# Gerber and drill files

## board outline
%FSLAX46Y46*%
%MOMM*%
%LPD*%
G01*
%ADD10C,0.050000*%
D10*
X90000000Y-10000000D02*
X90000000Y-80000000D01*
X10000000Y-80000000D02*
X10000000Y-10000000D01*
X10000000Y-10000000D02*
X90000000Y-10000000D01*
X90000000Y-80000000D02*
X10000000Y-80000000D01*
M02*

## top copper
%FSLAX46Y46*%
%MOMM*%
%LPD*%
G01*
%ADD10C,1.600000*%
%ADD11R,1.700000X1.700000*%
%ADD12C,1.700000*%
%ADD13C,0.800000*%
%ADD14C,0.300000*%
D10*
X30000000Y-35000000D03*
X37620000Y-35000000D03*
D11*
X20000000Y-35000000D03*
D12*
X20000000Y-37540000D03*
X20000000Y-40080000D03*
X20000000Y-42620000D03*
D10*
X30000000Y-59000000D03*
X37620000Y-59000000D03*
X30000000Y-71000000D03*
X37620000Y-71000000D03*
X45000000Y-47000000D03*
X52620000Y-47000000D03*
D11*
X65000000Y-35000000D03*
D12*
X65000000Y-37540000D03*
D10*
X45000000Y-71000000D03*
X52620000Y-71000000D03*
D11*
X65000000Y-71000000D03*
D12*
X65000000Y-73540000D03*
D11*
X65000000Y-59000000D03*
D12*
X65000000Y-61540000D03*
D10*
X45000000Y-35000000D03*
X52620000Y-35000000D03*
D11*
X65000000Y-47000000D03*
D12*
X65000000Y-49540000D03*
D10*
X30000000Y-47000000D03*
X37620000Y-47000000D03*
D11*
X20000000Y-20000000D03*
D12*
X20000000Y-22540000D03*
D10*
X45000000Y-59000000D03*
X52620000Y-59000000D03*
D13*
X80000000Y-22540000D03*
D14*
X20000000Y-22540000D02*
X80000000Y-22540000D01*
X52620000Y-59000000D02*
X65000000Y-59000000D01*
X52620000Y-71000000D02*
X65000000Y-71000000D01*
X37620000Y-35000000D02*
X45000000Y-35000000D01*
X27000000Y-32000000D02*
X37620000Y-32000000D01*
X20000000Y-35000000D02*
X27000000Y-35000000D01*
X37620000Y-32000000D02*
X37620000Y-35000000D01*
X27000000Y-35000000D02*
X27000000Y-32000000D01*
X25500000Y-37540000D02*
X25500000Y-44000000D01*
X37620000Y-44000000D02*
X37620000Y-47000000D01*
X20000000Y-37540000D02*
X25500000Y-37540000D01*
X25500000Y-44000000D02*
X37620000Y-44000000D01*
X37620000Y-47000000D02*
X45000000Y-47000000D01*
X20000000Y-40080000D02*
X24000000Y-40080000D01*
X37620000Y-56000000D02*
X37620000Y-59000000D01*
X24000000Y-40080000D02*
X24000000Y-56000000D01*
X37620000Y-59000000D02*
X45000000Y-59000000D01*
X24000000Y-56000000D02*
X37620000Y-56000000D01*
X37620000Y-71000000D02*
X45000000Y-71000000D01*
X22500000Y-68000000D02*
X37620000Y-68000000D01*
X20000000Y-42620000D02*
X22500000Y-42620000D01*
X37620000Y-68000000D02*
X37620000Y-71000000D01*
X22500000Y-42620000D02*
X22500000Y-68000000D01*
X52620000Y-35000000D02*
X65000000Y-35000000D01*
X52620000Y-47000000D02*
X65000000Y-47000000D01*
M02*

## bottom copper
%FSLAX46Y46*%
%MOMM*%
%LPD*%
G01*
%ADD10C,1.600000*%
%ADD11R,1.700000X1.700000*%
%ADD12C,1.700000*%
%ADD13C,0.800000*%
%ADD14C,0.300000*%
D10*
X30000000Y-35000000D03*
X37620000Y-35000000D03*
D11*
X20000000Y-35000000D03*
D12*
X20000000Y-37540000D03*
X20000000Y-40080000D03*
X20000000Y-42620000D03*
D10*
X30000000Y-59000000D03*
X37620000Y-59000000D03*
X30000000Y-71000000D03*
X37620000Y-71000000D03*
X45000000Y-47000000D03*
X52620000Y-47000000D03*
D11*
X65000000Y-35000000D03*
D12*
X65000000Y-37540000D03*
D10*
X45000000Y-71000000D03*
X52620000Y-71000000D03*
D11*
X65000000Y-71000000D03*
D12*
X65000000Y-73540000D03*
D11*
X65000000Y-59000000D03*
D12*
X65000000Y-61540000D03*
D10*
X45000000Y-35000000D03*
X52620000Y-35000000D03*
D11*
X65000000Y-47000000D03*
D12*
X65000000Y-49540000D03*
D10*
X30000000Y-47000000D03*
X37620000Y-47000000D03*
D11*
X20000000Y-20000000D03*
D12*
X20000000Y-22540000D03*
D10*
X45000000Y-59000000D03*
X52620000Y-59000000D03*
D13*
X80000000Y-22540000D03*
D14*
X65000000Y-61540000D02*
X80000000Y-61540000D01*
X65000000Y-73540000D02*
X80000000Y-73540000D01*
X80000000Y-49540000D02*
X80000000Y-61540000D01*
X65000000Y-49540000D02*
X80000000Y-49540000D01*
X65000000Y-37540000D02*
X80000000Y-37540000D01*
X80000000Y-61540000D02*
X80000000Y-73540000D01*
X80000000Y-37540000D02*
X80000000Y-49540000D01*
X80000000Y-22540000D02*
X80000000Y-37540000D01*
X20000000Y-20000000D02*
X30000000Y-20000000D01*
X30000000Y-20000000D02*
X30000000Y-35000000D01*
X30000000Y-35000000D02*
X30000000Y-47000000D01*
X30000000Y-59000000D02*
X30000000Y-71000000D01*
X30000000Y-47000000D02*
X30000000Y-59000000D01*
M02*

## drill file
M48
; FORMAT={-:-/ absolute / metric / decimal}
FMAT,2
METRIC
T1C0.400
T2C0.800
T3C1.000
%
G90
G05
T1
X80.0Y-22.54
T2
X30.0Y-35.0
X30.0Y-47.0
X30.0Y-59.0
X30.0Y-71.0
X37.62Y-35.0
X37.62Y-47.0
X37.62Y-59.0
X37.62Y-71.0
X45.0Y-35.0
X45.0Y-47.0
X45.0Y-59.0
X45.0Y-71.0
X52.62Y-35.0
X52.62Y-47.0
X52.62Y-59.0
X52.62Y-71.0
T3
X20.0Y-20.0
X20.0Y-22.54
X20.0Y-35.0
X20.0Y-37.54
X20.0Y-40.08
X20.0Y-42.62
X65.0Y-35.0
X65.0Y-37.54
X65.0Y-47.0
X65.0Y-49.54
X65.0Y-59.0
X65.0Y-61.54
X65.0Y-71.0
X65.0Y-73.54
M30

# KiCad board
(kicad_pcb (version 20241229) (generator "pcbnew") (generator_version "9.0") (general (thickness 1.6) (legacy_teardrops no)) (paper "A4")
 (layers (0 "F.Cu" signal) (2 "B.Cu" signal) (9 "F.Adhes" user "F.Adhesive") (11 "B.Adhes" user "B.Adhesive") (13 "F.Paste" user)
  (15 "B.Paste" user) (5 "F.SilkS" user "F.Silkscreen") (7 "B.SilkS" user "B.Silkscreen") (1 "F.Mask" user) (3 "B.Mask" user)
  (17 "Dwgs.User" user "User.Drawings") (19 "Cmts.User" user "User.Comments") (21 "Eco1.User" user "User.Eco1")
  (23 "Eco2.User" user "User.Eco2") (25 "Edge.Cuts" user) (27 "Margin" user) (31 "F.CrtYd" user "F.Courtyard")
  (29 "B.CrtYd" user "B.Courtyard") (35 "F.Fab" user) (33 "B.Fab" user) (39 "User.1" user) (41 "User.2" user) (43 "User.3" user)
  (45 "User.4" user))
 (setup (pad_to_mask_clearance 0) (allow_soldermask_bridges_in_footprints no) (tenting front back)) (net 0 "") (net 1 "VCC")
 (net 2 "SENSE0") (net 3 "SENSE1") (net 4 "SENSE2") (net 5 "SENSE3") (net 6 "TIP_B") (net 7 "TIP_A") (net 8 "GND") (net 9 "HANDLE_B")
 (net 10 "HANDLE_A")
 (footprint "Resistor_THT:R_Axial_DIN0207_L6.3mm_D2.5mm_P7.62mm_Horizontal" (layer "F.Cu") (at 30 35)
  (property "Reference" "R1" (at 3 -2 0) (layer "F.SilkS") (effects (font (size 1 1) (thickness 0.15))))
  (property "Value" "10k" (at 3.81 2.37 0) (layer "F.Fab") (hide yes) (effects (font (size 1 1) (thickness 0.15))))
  (pad "1" thru_hole circle (at 0 0) (size 1.6 1.6) (drill 0.8) (layers "*.Cu" "*.Mask") (remove_unused_layers no) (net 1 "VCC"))
  (pad "2" thru_hole circle (at 7.62 0) (size 1.6 1.6) (drill 0.8) (layers "*.Cu" "*.Mask") (remove_unused_layers no) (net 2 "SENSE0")))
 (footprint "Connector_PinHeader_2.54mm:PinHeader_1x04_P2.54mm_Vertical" (layer "F.Cu") (at 20 35)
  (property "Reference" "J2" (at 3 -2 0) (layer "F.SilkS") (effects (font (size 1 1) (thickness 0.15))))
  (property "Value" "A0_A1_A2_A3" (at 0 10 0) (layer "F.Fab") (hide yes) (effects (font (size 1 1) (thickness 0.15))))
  (pad "1" thru_hole rect (at 0 0) (size 1.7 1.7) (drill 1) (layers "*.Cu" "*.Mask") (remove_unused_layers no) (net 2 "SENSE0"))
  (pad "2" thru_hole circle (at 0 2.54) (size 1.7 1.7) (drill 1) (layers "*.Cu" "*.Mask") (remove_unused_layers no) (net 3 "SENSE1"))
  (pad "3" thru_hole circle (at 0 5.08) (size 1.7 1.7) (drill 1) (layers "*.Cu" "*.Mask") (remove_unused_layers no) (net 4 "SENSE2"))
  (pad "4" thru_hole circle (at 0 7.62) (size 1.7 1.7) (drill 1) (layers "*.Cu" "*.Mask") (remove_unused_layers no) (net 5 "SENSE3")))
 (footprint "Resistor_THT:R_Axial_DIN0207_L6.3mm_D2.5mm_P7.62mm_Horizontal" (layer "F.Cu") (at 30 59)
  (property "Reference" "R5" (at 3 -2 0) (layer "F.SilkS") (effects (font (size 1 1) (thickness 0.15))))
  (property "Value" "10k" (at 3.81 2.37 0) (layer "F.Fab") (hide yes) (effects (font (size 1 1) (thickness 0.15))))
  (pad "1" thru_hole circle (at 0 0) (size 1.6 1.6) (drill 0.8) (layers "*.Cu" "*.Mask") (remove_unused_layers no) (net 1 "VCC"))
  (pad "2" thru_hole circle (at 7.62 0) (size 1.6 1.6) (drill 0.8) (layers "*.Cu" "*.Mask") (remove_unused_layers no) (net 4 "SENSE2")))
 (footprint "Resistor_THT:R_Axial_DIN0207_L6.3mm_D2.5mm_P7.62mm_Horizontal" (layer "F.Cu") (at 30 71)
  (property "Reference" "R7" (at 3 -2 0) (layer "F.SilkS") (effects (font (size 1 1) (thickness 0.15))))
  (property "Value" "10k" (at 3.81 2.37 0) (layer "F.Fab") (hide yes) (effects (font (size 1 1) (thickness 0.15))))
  (pad "1" thru_hole circle (at 0 0) (size 1.6 1.6) (drill 0.8) (layers "*.Cu" "*.Mask") (remove_unused_layers no) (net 1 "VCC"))
  (pad "2" thru_hole circle (at 7.62 0) (size 1.6 1.6) (drill 0.8) (layers "*.Cu" "*.Mask") (remove_unused_layers no) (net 5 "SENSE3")))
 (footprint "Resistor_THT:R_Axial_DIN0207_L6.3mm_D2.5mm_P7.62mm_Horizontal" (layer "F.Cu") (at 45 47)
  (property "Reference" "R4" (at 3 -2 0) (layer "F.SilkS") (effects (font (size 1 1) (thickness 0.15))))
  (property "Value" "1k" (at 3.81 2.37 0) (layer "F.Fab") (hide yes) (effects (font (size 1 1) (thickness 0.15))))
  (pad "1" thru_hole circle (at 0 0) (size 1.6 1.6) (drill 0.8) (layers "*.Cu" "*.Mask") (remove_unused_layers no) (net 3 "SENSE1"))
  (pad "2" thru_hole circle (at 7.62 0) (size 1.6 1.6) (drill 0.8) (layers "*.Cu" "*.Mask") (remove_unused_layers no) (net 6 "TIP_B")))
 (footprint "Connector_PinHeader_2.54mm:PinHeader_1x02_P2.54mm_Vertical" (layer "F.Cu") (at 65 35)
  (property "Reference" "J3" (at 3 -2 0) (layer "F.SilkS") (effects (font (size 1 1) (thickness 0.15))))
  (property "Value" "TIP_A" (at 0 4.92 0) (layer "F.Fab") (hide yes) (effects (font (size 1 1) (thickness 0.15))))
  (pad "1" thru_hole rect (at 0 0) (size 1.7 1.7) (drill 1) (layers "*.Cu" "*.Mask") (remove_unused_layers no) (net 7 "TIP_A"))
  (pad "2" thru_hole circle (at 0 2.54) (size 1.7 1.7) (drill 1) (layers "*.Cu" "*.Mask") (remove_unused_layers no) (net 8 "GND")))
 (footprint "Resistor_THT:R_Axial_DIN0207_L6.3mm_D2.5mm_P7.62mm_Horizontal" (layer "F.Cu") (at 45 71)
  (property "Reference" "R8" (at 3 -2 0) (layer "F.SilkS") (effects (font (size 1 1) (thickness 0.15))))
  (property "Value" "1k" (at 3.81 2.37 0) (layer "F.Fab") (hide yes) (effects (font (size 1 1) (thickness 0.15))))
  (pad "1" thru_hole circle (at 0 0) (size 1.6 1.6) (drill 0.8) (layers "*.Cu" "*.Mask") (remove_unused_layers no) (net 5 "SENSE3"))
  (pad "2" thru_hole circle (at 7.62 0) (size 1.6 1.6) (drill 0.8) (layers "*.Cu" "*.Mask") (remove_unused_layers no) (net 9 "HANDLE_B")))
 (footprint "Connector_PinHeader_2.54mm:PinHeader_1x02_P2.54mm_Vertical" (layer "F.Cu") (at 65 71)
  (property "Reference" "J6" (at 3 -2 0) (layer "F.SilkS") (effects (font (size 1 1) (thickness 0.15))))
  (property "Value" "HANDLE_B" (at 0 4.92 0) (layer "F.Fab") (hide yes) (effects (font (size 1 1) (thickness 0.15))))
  (pad "1" thru_hole rect (at 0 0) (size 1.7 1.7) (drill 1) (layers "*.Cu" "*.Mask") (remove_unused_layers no) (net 9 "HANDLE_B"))
  (pad "2" thru_hole circle (at 0 2.54) (size 1.7 1.7) (drill 1) (layers "*.Cu" "*.Mask") (remove_unused_layers no) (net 8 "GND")))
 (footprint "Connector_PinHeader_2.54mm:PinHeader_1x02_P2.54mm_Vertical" (layer "F.Cu") (at 65 59)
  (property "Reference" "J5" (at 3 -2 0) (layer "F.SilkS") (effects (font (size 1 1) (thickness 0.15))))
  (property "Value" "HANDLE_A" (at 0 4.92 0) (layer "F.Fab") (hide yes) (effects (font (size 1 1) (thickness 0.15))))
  (pad "1" thru_hole rect (at 0 0) (size 1.7 1.7) (drill 1) (layers "*.Cu" "*.Mask") (remove_unused_layers no) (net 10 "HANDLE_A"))
  (pad "2" thru_hole circle (at 0 2.54) (size 1.7 1.7) (drill 1) (layers "*.Cu" "*.Mask") (remove_unused_layers no) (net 8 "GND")))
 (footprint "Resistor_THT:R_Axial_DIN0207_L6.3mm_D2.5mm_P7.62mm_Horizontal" (layer "F.Cu") (at 45 35)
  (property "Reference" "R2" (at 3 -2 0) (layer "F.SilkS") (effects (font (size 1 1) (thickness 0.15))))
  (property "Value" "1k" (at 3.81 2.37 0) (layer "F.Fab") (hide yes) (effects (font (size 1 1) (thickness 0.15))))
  (pad "1" thru_hole circle (at 0 0) (size 1.6 1.6) (drill 0.8) (layers "*.Cu" "*.Mask") (remove_unused_layers no) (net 2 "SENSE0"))
  (pad "2" thru_hole circle (at 7.62 0) (size 1.6 1.6) (drill 0.8) (layers "*.Cu" "*.Mask") (remove_unused_layers no) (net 7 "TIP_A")))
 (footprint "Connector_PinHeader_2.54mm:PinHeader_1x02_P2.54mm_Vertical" (layer "F.Cu") (at 65 47)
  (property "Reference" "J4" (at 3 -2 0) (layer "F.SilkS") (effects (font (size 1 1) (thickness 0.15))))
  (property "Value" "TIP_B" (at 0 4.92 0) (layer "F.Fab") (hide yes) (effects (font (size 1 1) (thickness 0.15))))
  (pad "1" thru_hole rect (at 0 0) (size 1.7 1.7) (drill 1) (layers "*.Cu" "*.Mask") (remove_unused_layers no) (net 6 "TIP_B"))
  (pad "2" thru_hole circle (at 0 2.54) (size 1.7 1.7) (drill 1) (layers "*.Cu" "*.Mask") (remove_unused_layers no) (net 8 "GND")))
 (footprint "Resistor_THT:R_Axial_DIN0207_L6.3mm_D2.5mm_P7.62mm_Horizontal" (layer "F.Cu") (at 30 47)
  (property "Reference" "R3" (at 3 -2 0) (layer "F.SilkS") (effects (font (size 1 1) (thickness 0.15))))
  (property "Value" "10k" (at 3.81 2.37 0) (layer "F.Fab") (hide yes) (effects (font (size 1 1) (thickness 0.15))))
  (pad "1" thru_hole circle (at 0 0) (size 1.6 1.6) (drill 0.8) (layers "*.Cu" "*.Mask") (remove_unused_layers no) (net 1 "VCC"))
  (pad "2" thru_hole circle (at 7.62 0) (size 1.6 1.6) (drill 0.8) (layers "*.Cu" "*.Mask") (remove_unused_layers no) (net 3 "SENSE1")))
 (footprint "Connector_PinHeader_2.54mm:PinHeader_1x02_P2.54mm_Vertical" (layer "F.Cu") (at 20 20)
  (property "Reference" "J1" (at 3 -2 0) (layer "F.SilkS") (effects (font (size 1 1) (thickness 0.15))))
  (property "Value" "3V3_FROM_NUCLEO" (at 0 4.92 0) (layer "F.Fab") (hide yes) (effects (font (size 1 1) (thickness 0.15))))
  (pad "1" thru_hole rect (at 0 0) (size 1.7 1.7) (drill 1) (layers "*.Cu" "*.Mask") (remove_unused_layers no) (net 1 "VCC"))
  (pad "2" thru_hole circle (at 0 2.54) (size 1.7 1.7) (drill 1) (layers "*.Cu" "*.Mask") (remove_unused_layers no) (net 8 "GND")))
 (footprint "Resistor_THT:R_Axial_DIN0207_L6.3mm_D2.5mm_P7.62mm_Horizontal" (layer "F.Cu") (at 45 59)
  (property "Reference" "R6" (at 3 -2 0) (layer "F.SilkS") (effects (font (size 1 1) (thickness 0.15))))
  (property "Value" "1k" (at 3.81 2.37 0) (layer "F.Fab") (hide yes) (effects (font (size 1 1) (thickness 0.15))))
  (pad "1" thru_hole circle (at 0 0) (size 1.6 1.6) (drill 0.8) (layers "*.Cu" "*.Mask") (remove_unused_layers no) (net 4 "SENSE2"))
  (pad "2" thru_hole circle (at 7.62 0) (size 1.6 1.6) (drill 0.8) (layers "*.Cu" "*.Mask") (remove_unused_layers no) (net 10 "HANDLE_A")))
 (gr_line (start 90 10) (end 90 80) (stroke (width 0.05) (type default)) (layer "Edge.Cuts"))
 (gr_line (start 10 80) (end 10 10) (stroke (width 0.05) (type default)) (layer "Edge.Cuts"))
 (gr_line (start 10 10) (end 90 10) (stroke (width 0.05) (type default)) (layer "Edge.Cuts"))
 (gr_line (start 90 80) (end 10 80) (stroke (width 0.05) (type default)) (layer "Edge.Cuts"))
 (segment (start 20 22.54) (end 80 22.54) (width 0.3) (layer "F.Cu") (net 8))
 (via (at 80 22.54) (size 0.8) (drill 0.4) (layers "F.Cu" "B.Cu") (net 8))
 (segment (start 65 61.54) (end 80 61.54) (width 0.3) (layer "B.Cu") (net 8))
 (segment (start 65 73.54) (end 80 73.54) (width 0.3) (layer "B.Cu") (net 8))
 (segment (start 80 49.54) (end 80 61.54) (width 0.3) (layer "B.Cu") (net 8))
 (segment (start 65 49.54) (end 80 49.54) (width 0.3) (layer "B.Cu") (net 8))
 (segment (start 65 37.54) (end 80 37.54) (width 0.3) (layer "B.Cu") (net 8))
 (segment (start 80 61.54) (end 80 73.54) (width 0.3) (layer "B.Cu") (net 8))
 (segment (start 80 37.54) (end 80 49.54) (width 0.3) (layer "B.Cu") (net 8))
 (segment (start 80 22.54) (end 80 37.54) (width 0.3) (layer "B.Cu") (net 8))
 (segment (start 52.62 59) (end 65 59) (width 0.3) (layer "F.Cu") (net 10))
 (segment (start 52.62 71) (end 65 71) (width 0.3) (layer "F.Cu") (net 9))
 (segment (start 37.62 35) (end 45 35) (width 0.3) (layer "F.Cu") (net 2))
 (segment (start 27 32) (end 37.62 32) (width 0.3) (layer "F.Cu") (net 2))
 (segment (start 20 35) (end 27 35) (width 0.3) (layer "F.Cu") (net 2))
 (segment (start 37.62 32) (end 37.62 35) (width 0.3) (layer "F.Cu") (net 2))
 (segment (start 27 35) (end 27 32) (width 0.3) (layer "F.Cu") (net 2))
 (segment (start 25.5 37.54) (end 25.5 44) (width 0.3) (layer "F.Cu") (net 3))
 (segment (start 37.62 44) (end 37.62 47) (width 0.3) (layer "F.Cu") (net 3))
 (segment (start 20 37.54) (end 25.5 37.54) (width 0.3) (layer "F.Cu") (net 3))
 (segment (start 25.5 44) (end 37.62 44) (width 0.3) (layer "F.Cu") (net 3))
 (segment (start 37.62 47) (end 45 47) (width 0.3) (layer "F.Cu") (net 3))
 (segment (start 20 40.08) (end 24 40.08) (width 0.3) (layer "F.Cu") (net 4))
 (segment (start 37.62 56) (end 37.62 59) (width 0.3) (layer "F.Cu") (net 4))
 (segment (start 24 40.08) (end 24 56) (width 0.3) (layer "F.Cu") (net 4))
 (segment (start 37.62 59) (end 45 59) (width 0.3) (layer "F.Cu") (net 4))
 (segment (start 24 56) (end 37.62 56) (width 0.3) (layer "F.Cu") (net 4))
 (segment (start 37.62 71) (end 45 71) (width 0.3) (layer "F.Cu") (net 5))
 (segment (start 22.5 68) (end 37.62 68) (width 0.3) (layer "F.Cu") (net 5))
 (segment (start 20 42.62) (end 22.5 42.62) (width 0.3) (layer "F.Cu") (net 5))
 (segment (start 37.62 68) (end 37.62 71) (width 0.3) (layer "F.Cu") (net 5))
 (segment (start 22.5 42.62) (end 22.5 68) (width 0.3) (layer "F.Cu") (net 5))
 (segment (start 52.62 35) (end 65 35) (width 0.3) (layer "F.Cu") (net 7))
 (segment (start 52.62 47) (end 65 47) (width 0.3) (layer "F.Cu") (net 6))
 (segment (start 20 20) (end 30 20) (width 0.3) (layer "B.Cu") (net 1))
 (segment (start 30 20) (end 30 35) (width 0.3) (layer "B.Cu") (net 1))
 (segment (start 30 35) (end 30 47) (width 0.3) (layer "B.Cu") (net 1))
 (segment (start 30 59) (end 30 71) (width 0.3) (layer "B.Cu") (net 1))
 (segment (start 30 47) (end 30 59) (width 0.3) (layer "B.Cu") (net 1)))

